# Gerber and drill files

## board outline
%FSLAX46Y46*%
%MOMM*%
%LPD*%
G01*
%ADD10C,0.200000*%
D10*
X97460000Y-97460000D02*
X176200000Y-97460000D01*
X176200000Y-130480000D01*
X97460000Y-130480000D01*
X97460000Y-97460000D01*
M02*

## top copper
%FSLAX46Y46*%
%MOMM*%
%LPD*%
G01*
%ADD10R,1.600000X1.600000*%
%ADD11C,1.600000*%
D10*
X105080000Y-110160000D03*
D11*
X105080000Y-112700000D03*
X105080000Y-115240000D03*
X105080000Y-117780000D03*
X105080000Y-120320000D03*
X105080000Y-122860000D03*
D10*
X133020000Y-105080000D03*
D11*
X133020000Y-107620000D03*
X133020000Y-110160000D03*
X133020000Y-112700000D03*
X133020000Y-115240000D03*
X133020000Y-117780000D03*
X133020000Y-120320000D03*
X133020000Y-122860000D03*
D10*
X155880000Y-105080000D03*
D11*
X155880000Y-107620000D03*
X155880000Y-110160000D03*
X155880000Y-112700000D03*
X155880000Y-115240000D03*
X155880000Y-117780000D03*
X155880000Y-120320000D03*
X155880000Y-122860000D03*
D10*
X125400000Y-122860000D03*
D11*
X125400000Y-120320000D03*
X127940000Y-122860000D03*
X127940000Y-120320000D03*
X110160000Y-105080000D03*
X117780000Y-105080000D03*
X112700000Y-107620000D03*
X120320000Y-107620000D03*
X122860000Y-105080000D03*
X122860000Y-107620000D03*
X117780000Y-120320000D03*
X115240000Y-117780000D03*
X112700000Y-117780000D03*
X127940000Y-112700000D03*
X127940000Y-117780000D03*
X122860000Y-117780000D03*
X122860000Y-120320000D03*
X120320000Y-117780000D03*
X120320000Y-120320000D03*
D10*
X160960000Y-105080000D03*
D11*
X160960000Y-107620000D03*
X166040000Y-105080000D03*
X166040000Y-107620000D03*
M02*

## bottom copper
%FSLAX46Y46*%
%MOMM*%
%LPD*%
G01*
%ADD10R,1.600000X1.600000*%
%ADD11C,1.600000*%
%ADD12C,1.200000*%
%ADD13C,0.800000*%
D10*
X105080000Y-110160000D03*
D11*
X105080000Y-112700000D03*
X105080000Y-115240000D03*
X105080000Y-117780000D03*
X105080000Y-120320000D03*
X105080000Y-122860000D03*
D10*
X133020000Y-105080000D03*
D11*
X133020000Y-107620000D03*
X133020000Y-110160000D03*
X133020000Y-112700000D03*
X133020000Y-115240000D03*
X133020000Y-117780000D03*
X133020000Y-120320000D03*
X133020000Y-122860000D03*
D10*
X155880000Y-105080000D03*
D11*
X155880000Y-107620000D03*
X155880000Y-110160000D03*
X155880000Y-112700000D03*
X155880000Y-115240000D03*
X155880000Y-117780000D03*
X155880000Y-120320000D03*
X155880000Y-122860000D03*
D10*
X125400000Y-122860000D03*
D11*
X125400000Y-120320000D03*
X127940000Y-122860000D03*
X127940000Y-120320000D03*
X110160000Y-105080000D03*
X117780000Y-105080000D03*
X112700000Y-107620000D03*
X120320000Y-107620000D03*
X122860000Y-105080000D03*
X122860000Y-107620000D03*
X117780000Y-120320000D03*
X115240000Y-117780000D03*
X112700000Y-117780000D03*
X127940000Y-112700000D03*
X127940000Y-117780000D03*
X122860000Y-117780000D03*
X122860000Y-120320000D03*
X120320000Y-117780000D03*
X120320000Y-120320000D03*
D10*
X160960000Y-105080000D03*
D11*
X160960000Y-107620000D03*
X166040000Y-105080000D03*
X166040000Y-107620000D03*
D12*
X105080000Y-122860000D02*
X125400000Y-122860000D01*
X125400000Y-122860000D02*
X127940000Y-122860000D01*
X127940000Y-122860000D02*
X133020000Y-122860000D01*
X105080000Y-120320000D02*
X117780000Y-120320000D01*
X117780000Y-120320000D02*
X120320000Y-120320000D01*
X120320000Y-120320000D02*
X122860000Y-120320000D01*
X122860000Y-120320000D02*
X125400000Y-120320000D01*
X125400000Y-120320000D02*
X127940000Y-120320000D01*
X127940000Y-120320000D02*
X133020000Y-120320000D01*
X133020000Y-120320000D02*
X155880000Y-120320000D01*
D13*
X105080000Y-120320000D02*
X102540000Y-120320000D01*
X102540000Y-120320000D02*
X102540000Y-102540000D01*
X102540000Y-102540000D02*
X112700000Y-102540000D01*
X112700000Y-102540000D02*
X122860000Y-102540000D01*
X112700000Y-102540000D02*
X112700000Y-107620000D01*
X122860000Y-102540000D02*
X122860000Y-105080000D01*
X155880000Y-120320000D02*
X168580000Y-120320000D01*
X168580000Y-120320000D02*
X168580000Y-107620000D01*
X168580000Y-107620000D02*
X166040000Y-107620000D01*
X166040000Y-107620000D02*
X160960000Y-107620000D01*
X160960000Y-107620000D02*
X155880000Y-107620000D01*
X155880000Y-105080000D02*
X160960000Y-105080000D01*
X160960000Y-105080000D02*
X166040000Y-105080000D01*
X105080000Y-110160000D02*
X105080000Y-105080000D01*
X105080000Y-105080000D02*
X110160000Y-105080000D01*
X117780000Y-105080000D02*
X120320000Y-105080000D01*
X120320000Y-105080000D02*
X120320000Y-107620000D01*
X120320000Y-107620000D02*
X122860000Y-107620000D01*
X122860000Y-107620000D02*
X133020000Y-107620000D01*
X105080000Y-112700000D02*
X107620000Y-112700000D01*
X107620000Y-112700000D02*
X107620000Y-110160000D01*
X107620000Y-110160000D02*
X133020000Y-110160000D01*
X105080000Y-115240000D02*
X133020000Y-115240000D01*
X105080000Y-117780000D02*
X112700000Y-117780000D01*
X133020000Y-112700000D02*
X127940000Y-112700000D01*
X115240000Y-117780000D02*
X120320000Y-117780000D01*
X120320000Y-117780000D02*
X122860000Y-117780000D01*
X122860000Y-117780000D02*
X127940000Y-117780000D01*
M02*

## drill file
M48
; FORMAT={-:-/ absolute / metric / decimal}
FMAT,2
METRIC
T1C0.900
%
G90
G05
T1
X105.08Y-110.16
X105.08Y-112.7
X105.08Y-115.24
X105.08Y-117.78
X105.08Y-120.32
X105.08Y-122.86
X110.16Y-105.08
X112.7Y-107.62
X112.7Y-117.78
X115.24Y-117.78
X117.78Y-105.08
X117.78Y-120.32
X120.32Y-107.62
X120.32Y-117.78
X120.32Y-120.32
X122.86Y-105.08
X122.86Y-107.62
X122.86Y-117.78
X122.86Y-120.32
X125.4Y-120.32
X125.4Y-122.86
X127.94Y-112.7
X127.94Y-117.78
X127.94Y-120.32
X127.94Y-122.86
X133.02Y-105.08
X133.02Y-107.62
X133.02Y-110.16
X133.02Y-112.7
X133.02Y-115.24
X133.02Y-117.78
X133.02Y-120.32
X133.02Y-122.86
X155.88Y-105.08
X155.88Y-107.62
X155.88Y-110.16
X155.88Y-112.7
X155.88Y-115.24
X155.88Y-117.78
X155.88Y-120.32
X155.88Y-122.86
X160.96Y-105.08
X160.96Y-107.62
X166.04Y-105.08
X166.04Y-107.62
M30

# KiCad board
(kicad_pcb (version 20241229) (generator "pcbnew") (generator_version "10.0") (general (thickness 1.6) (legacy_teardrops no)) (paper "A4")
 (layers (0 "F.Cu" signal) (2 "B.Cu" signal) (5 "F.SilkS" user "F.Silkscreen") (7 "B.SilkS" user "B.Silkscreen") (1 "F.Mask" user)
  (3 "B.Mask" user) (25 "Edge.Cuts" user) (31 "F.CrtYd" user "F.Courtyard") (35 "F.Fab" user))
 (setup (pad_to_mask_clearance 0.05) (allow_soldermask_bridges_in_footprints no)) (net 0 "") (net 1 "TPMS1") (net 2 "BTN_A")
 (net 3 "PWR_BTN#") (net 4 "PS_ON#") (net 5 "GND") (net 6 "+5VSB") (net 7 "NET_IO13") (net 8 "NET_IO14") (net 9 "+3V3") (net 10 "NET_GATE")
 (gr_rect (start 97.46 97.46) (end 176.2 130.48) (stroke (width 0.2) (type solid)) (fill none) (layer "Edge.Cuts"))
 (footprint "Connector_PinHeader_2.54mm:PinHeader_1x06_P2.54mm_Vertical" (layer "F.Cu") (at 0 0)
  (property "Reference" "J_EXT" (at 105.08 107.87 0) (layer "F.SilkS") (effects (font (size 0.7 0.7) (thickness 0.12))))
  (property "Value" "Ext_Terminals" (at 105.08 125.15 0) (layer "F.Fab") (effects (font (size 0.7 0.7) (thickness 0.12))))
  (pad "1" thru_hole rect (at 105.08 110.16) (size 1.6 1.6) (drill 0.9) (layers "*.Cu" "*.Mask") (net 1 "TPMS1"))
  (pad "2" thru_hole circle (at 105.08 112.7) (size 1.6 1.6) (drill 0.9) (layers "*.Cu" "*.Mask") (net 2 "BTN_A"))
  (pad "3" thru_hole circle (at 105.08 115.24) (size 1.6 1.6) (drill 0.9) (layers "*.Cu" "*.Mask") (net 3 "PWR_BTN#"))
  (pad "4" thru_hole circle (at 105.08 117.78) (size 1.6 1.6) (drill 0.9) (layers "*.Cu" "*.Mask") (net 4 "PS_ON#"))
  (pad "5" thru_hole circle (at 105.08 120.32) (size 1.6 1.6) (drill 0.9) (layers "*.Cu" "*.Mask") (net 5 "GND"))
  (pad "6" thru_hole circle (at 105.08 122.86) (size 1.6 1.6) (drill 0.9) (layers "*.Cu" "*.Mask") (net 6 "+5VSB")))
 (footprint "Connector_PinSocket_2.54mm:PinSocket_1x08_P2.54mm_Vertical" (layer "F.Cu") (at 0 0)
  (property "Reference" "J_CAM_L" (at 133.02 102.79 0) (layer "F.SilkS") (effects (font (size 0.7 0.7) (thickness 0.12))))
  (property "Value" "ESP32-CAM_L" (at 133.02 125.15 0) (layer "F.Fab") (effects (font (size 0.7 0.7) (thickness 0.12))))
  (pad "1" thru_hole rect (at 133.02 105.08) (size 1.6 1.6) (drill 0.9) (layers "*.Cu" "*.Mask") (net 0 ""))
  (pad "2" thru_hole circle (at 133.02 107.62) (size 1.6 1.6) (drill 0.9) (layers "*.Cu" "*.Mask") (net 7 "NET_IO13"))
  (pad "3" thru_hole circle (at 133.02 110.16) (size 1.6 1.6) (drill 0.9) (layers "*.Cu" "*.Mask") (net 2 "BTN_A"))
  (pad "4" thru_hole circle (at 133.02 112.7) (size 1.6 1.6) (drill 0.9) (layers "*.Cu" "*.Mask") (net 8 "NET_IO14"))
  (pad "5" thru_hole circle (at 133.02 115.24) (size 1.6 1.6) (drill 0.9) (layers "*.Cu" "*.Mask") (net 3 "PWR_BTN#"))
  (pad "6" thru_hole circle (at 133.02 117.78) (size 1.6 1.6) (drill 0.9) (layers "*.Cu" "*.Mask") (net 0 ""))
  (pad "7" thru_hole circle (at 133.02 120.32) (size 1.6 1.6) (drill 0.9) (layers "*.Cu" "*.Mask") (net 5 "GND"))
  (pad "8" thru_hole circle (at 133.02 122.86) (size 1.6 1.6) (drill 0.9) (layers "*.Cu" "*.Mask") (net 6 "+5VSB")))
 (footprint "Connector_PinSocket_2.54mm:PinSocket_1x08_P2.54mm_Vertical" (layer "F.Cu") (at 0 0)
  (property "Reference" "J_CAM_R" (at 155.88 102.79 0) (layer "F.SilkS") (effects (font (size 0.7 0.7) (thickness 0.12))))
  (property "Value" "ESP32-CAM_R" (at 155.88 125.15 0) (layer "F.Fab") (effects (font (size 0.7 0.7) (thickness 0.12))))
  (pad "1" thru_hole rect (at 155.88 105.08) (size 1.6 1.6) (drill 0.9) (layers "*.Cu" "*.Mask") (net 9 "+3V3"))
  (pad "2" thru_hole circle (at 155.88 107.62) (size 1.6 1.6) (drill 0.9) (layers "*.Cu" "*.Mask") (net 5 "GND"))
  (pad "3" thru_hole circle (at 155.88 110.16) (size 1.6 1.6) (drill 0.9) (layers "*.Cu" "*.Mask") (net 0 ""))
  (pad "4" thru_hole circle (at 155.88 112.7) (size 1.6 1.6) (drill 0.9) (layers "*.Cu" "*.Mask") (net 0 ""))
  (pad "5" thru_hole circle (at 155.88 115.24) (size 1.6 1.6) (drill 0.9) (layers "*.Cu" "*.Mask") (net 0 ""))
  (pad "6" thru_hole circle (at 155.88 117.78) (size 1.6 1.6) (drill 0.9) (layers "*.Cu" "*.Mask") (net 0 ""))
  (pad "7" thru_hole circle (at 155.88 120.32) (size 1.6 1.6) (drill 0.9) (layers "*.Cu" "*.Mask") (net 5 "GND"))
  (pad "8" thru_hole circle (at 155.88 122.86) (size 1.6 1.6) (drill 0.9) (layers "*.Cu" "*.Mask") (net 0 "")))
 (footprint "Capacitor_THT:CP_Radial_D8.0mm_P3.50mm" (layer "F.Cu") (at 0 0)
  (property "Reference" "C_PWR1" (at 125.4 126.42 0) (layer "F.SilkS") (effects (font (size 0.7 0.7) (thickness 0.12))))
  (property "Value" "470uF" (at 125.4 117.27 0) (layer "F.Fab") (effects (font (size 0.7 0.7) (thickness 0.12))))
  (pad "1" thru_hole rect (at 125.4 122.86) (size 1.6 1.6) (drill 0.9) (layers "*.Cu" "*.Mask") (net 6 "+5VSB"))
  (pad "2" thru_hole circle (at 125.4 120.32) (size 1.6 1.6) (drill 0.9) (layers "*.Cu" "*.Mask") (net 5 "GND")))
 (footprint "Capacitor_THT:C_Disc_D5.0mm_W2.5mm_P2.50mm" (layer "F.Cu") (at 0 0)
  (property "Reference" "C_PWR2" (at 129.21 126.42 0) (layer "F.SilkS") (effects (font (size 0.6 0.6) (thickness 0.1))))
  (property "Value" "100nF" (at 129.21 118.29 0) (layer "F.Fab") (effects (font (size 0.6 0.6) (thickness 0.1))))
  (pad "1" thru_hole circle (at 127.94 122.86) (size 1.6 1.6) (drill 0.9) (layers "*.Cu" "*.Mask") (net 6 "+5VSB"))
  (pad "2" thru_hole circle (at 127.94 120.32) (size 1.6 1.6) (drill 0.9) (layers "*.Cu" "*.Mask") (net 5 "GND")))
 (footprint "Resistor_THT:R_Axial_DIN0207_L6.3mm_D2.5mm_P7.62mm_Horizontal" (layer "F.Cu") (at 0 0)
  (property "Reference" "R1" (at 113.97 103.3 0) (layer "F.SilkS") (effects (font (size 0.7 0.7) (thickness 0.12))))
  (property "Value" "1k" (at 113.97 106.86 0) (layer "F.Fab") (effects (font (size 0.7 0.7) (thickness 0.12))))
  (pad "1" thru_hole circle (at 110.16 105.08) (size 1.6 1.6) (drill 0.9) (layers "*.Cu" "*.Mask") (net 1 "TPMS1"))
  (pad "2" thru_hole circle (at 117.78 105.08) (size 1.6 1.6) (drill 0.9) (layers "*.Cu" "*.Mask") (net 7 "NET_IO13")))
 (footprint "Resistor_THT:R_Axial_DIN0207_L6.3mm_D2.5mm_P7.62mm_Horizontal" (layer "F.Cu") (at 0 0)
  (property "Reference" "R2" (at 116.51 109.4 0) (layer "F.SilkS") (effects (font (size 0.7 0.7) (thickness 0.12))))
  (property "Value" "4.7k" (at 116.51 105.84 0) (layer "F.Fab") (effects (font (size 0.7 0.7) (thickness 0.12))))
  (pad "1" thru_hole circle (at 112.7 107.62) (size 1.6 1.6) (drill 0.9) (layers "*.Cu" "*.Mask") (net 5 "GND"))
  (pad "2" thru_hole circle (at 120.32 107.62) (size 1.6 1.6) (drill 0.9) (layers "*.Cu" "*.Mask") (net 7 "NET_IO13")))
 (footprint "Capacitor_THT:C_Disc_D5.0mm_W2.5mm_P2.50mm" (layer "F.Cu") (at 0 0)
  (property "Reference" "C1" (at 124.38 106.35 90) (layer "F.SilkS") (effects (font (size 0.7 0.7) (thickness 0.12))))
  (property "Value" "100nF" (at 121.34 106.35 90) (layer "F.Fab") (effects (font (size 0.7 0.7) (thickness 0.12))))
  (pad "1" thru_hole circle (at 122.86 105.08) (size 1.6 1.6) (drill 0.9) (layers "*.Cu" "*.Mask") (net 5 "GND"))
  (pad "2" thru_hole circle (at 122.86 107.62) (size 1.6 1.6) (drill 0.9) (layers "*.Cu" "*.Mask") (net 7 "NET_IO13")))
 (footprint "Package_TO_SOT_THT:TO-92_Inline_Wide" (layer "F.Cu") (at 0 0)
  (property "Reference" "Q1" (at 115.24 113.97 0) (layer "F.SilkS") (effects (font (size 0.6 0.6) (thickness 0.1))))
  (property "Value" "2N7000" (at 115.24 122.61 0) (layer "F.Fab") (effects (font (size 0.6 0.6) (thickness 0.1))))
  (pad "1" thru_hole circle (at 117.78 120.32) (size 1.6 1.6) (drill 0.9) (layers "*.Cu" "*.Mask") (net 5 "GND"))
  (pad "2" thru_hole circle (at 115.24 117.78) (size 1.6 1.6) (drill 0.9) (layers "*.Cu" "*.Mask") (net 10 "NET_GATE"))
  (pad "3" thru_hole circle (at 112.7 117.78) (size 1.6 1.6) (drill 0.9) (layers "*.Cu" "*.Mask") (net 4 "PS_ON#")))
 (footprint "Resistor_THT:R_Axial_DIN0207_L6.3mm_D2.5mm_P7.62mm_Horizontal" (layer "F.Cu") (at 0 0)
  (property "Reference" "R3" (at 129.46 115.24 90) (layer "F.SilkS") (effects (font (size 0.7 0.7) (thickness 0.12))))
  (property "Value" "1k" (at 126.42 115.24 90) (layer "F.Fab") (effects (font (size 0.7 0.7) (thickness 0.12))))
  (pad "1" thru_hole circle (at 127.94 112.7) (size 1.6 1.6) (drill 0.9) (layers "*.Cu" "*.Mask") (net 8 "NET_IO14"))
  (pad "2" thru_hole circle (at 127.94 117.78) (size 1.6 1.6) (drill 0.9) (layers "*.Cu" "*.Mask") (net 10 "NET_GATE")))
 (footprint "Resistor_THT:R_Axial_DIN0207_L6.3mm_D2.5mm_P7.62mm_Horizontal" (layer "F.Cu") (at 0 0)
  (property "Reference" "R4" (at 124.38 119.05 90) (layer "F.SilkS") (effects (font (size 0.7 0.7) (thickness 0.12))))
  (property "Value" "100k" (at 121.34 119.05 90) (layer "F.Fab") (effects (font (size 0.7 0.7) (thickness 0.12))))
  (pad "1" thru_hole circle (at 122.86 117.78) (size 1.6 1.6) (drill 0.9) (layers "*.Cu" "*.Mask") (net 10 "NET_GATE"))
  (pad "2" thru_hole circle (at 122.86 120.32) (size 1.6 1.6) (drill 0.9) (layers "*.Cu" "*.Mask") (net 5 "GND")))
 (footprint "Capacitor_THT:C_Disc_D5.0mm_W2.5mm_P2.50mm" (layer "F.Cu") (at 0 0)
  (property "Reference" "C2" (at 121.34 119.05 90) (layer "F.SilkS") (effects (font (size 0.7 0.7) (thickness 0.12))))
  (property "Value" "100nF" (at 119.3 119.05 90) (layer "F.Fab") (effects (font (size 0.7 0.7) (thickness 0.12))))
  (pad "1" thru_hole circle (at 120.32 117.78) (size 1.6 1.6) (drill 0.9) (layers "*.Cu" "*.Mask") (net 10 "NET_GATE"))
  (pad "2" thru_hole circle (at 120.32 120.32) (size 1.6 1.6) (drill 0.9) (layers "*.Cu" "*.Mask") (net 5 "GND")))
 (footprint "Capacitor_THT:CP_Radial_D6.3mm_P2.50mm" (layer "F.Cu") (at 0 0)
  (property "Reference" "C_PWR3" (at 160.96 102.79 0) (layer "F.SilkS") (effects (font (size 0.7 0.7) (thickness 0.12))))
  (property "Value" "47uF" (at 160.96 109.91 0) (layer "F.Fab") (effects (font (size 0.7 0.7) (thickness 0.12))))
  (pad "1" thru_hole rect (at 160.96 105.08) (size 1.6 1.6) (drill 0.9) (layers "*.Cu" "*.Mask") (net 9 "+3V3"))
  (pad "2" thru_hole circle (at 160.96 107.62) (size 1.6 1.6) (drill 0.9) (layers "*.Cu" "*.Mask") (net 5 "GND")))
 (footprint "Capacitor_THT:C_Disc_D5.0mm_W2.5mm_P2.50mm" (layer "F.Cu") (at 0 0)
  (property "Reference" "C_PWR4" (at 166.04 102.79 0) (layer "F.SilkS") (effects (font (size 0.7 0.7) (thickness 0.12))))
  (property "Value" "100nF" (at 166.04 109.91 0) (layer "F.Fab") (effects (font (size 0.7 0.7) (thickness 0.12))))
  (pad "1" thru_hole circle (at 166.04 105.08) (size 1.6 1.6) (drill 0.9) (layers "*.Cu" "*.Mask") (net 9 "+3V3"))
  (pad "2" thru_hole circle (at 166.04 107.62) (size 1.6 1.6) (drill 0.9) (layers "*.Cu" "*.Mask") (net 5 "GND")))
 (segment (start 105.08 122.86) (end 125.4 122.86) (width 1.2) (layer "B.Cu") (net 6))
 (segment (start 125.4 122.86) (end 127.94 122.86) (width 1.2) (layer "B.Cu") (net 6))
 (segment (start 127.94 122.86) (end 133.02 122.86) (width 1.2) (layer "B.Cu") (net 6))
 (segment (start 105.08 120.32) (end 117.78 120.32) (width 1.2) (layer "B.Cu") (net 5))
 (segment (start 117.78 120.32) (end 120.32 120.32) (width 1.2) (layer "B.Cu") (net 5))
 (segment (start 120.32 120.32) (end 122.86 120.32) (width 1.2) (layer "B.Cu") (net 5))
 (segment (start 122.86 120.32) (end 125.4 120.32) (width 1.2) (layer "B.Cu") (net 5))
 (segment (start 125.4 120.32) (end 127.94 120.32) (width 1.2) (layer "B.Cu") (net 5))
 (segment (start 127.94 120.32) (end 133.02 120.32) (width 1.2) (layer "B.Cu") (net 5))
 (segment (start 133.02 120.32) (end 155.88 120.32) (width 1.2) (layer "B.Cu") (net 5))
 (segment (start 105.08 120.32) (end 102.54 120.32) (width 0.8) (layer "B.Cu") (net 5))
 (segment (start 102.54 120.32) (end 102.54 102.54) (width 0.8) (layer "B.Cu") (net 5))
 (segment (start 102.54 102.54) (end 112.7 102.54) (width 0.8) (layer "B.Cu") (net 5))
 (segment (start 112.7 102.54) (end 122.86 102.54) (width 0.8) (layer "B.Cu") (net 5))
 (segment (start 112.7 102.54) (end 112.7 107.62) (width 0.8) (layer "B.Cu") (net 5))
 (segment (start 122.86 102.54) (end 122.86 105.08) (width 0.8) (layer "B.Cu") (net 5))
 (segment (start 155.88 120.32) (end 168.58 120.32) (width 0.8) (layer "B.Cu") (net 5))
 (segment (start 168.58 120.32) (end 168.58 107.62) (width 0.8) (layer "B.Cu") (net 5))
 (segment (start 168.58 107.62) (end 166.04 107.62) (width 0.8) (layer "B.Cu") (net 5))
 (segment (start 166.04 107.62) (end 160.96 107.62) (width 0.8) (layer "B.Cu") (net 5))
 (segment (start 160.96 107.62) (end 155.88 107.62) (width 0.8) (layer "B.Cu") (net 5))
 (segment (start 155.88 105.08) (end 160.96 105.08) (width 0.8) (layer "B.Cu") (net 9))
 (segment (start 160.96 105.08) (end 166.04 105.08) (width 0.8) (layer "B.Cu") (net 9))
 (segment (start 105.08 110.16) (end 105.08 105.08) (width 0.8) (layer "B.Cu") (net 1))
 (segment (start 105.08 105.08) (end 110.16 105.08) (width 0.8) (layer "B.Cu") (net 1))
 (segment (start 117.78 105.08) (end 120.32 105.08) (width 0.8) (layer "B.Cu") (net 7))
 (segment (start 120.32 105.08) (end 120.32 107.62) (width 0.8) (layer "B.Cu") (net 7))
 (segment (start 120.32 107.62) (end 122.86 107.62) (width 0.8) (layer "B.Cu") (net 7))
 (segment (start 122.86 107.62) (end 133.02 107.62) (width 0.8) (layer "B.Cu") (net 7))
 (segment (start 105.08 112.7) (end 107.62 112.7) (width 0.8) (layer "B.Cu") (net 2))
 (segment (start 107.62 112.7) (end 107.62 110.16) (width 0.8) (layer "B.Cu") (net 2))
 (segment (start 107.62 110.16) (end 133.02 110.16) (width 0.8) (layer "B.Cu") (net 2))
 (segment (start 105.08 115.24) (end 133.02 115.24) (width 0.8) (layer "B.Cu") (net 3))
 (segment (start 105.08 117.78) (end 112.7 117.78) (width 0.8) (layer "B.Cu") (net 4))
 (segment (start 133.02 112.7) (end 127.94 112.7) (width 0.8) (layer "B.Cu") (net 8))
 (segment (start 115.24 117.78) (end 120.32 117.78) (width 0.8) (layer "B.Cu") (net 10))
 (segment (start 120.32 117.78) (end 122.86 117.78) (width 0.8) (layer "B.Cu") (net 10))
 (segment (start 122.86 117.78) (end 127.94 117.78) (width 0.8) (layer "B.Cu") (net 10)))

